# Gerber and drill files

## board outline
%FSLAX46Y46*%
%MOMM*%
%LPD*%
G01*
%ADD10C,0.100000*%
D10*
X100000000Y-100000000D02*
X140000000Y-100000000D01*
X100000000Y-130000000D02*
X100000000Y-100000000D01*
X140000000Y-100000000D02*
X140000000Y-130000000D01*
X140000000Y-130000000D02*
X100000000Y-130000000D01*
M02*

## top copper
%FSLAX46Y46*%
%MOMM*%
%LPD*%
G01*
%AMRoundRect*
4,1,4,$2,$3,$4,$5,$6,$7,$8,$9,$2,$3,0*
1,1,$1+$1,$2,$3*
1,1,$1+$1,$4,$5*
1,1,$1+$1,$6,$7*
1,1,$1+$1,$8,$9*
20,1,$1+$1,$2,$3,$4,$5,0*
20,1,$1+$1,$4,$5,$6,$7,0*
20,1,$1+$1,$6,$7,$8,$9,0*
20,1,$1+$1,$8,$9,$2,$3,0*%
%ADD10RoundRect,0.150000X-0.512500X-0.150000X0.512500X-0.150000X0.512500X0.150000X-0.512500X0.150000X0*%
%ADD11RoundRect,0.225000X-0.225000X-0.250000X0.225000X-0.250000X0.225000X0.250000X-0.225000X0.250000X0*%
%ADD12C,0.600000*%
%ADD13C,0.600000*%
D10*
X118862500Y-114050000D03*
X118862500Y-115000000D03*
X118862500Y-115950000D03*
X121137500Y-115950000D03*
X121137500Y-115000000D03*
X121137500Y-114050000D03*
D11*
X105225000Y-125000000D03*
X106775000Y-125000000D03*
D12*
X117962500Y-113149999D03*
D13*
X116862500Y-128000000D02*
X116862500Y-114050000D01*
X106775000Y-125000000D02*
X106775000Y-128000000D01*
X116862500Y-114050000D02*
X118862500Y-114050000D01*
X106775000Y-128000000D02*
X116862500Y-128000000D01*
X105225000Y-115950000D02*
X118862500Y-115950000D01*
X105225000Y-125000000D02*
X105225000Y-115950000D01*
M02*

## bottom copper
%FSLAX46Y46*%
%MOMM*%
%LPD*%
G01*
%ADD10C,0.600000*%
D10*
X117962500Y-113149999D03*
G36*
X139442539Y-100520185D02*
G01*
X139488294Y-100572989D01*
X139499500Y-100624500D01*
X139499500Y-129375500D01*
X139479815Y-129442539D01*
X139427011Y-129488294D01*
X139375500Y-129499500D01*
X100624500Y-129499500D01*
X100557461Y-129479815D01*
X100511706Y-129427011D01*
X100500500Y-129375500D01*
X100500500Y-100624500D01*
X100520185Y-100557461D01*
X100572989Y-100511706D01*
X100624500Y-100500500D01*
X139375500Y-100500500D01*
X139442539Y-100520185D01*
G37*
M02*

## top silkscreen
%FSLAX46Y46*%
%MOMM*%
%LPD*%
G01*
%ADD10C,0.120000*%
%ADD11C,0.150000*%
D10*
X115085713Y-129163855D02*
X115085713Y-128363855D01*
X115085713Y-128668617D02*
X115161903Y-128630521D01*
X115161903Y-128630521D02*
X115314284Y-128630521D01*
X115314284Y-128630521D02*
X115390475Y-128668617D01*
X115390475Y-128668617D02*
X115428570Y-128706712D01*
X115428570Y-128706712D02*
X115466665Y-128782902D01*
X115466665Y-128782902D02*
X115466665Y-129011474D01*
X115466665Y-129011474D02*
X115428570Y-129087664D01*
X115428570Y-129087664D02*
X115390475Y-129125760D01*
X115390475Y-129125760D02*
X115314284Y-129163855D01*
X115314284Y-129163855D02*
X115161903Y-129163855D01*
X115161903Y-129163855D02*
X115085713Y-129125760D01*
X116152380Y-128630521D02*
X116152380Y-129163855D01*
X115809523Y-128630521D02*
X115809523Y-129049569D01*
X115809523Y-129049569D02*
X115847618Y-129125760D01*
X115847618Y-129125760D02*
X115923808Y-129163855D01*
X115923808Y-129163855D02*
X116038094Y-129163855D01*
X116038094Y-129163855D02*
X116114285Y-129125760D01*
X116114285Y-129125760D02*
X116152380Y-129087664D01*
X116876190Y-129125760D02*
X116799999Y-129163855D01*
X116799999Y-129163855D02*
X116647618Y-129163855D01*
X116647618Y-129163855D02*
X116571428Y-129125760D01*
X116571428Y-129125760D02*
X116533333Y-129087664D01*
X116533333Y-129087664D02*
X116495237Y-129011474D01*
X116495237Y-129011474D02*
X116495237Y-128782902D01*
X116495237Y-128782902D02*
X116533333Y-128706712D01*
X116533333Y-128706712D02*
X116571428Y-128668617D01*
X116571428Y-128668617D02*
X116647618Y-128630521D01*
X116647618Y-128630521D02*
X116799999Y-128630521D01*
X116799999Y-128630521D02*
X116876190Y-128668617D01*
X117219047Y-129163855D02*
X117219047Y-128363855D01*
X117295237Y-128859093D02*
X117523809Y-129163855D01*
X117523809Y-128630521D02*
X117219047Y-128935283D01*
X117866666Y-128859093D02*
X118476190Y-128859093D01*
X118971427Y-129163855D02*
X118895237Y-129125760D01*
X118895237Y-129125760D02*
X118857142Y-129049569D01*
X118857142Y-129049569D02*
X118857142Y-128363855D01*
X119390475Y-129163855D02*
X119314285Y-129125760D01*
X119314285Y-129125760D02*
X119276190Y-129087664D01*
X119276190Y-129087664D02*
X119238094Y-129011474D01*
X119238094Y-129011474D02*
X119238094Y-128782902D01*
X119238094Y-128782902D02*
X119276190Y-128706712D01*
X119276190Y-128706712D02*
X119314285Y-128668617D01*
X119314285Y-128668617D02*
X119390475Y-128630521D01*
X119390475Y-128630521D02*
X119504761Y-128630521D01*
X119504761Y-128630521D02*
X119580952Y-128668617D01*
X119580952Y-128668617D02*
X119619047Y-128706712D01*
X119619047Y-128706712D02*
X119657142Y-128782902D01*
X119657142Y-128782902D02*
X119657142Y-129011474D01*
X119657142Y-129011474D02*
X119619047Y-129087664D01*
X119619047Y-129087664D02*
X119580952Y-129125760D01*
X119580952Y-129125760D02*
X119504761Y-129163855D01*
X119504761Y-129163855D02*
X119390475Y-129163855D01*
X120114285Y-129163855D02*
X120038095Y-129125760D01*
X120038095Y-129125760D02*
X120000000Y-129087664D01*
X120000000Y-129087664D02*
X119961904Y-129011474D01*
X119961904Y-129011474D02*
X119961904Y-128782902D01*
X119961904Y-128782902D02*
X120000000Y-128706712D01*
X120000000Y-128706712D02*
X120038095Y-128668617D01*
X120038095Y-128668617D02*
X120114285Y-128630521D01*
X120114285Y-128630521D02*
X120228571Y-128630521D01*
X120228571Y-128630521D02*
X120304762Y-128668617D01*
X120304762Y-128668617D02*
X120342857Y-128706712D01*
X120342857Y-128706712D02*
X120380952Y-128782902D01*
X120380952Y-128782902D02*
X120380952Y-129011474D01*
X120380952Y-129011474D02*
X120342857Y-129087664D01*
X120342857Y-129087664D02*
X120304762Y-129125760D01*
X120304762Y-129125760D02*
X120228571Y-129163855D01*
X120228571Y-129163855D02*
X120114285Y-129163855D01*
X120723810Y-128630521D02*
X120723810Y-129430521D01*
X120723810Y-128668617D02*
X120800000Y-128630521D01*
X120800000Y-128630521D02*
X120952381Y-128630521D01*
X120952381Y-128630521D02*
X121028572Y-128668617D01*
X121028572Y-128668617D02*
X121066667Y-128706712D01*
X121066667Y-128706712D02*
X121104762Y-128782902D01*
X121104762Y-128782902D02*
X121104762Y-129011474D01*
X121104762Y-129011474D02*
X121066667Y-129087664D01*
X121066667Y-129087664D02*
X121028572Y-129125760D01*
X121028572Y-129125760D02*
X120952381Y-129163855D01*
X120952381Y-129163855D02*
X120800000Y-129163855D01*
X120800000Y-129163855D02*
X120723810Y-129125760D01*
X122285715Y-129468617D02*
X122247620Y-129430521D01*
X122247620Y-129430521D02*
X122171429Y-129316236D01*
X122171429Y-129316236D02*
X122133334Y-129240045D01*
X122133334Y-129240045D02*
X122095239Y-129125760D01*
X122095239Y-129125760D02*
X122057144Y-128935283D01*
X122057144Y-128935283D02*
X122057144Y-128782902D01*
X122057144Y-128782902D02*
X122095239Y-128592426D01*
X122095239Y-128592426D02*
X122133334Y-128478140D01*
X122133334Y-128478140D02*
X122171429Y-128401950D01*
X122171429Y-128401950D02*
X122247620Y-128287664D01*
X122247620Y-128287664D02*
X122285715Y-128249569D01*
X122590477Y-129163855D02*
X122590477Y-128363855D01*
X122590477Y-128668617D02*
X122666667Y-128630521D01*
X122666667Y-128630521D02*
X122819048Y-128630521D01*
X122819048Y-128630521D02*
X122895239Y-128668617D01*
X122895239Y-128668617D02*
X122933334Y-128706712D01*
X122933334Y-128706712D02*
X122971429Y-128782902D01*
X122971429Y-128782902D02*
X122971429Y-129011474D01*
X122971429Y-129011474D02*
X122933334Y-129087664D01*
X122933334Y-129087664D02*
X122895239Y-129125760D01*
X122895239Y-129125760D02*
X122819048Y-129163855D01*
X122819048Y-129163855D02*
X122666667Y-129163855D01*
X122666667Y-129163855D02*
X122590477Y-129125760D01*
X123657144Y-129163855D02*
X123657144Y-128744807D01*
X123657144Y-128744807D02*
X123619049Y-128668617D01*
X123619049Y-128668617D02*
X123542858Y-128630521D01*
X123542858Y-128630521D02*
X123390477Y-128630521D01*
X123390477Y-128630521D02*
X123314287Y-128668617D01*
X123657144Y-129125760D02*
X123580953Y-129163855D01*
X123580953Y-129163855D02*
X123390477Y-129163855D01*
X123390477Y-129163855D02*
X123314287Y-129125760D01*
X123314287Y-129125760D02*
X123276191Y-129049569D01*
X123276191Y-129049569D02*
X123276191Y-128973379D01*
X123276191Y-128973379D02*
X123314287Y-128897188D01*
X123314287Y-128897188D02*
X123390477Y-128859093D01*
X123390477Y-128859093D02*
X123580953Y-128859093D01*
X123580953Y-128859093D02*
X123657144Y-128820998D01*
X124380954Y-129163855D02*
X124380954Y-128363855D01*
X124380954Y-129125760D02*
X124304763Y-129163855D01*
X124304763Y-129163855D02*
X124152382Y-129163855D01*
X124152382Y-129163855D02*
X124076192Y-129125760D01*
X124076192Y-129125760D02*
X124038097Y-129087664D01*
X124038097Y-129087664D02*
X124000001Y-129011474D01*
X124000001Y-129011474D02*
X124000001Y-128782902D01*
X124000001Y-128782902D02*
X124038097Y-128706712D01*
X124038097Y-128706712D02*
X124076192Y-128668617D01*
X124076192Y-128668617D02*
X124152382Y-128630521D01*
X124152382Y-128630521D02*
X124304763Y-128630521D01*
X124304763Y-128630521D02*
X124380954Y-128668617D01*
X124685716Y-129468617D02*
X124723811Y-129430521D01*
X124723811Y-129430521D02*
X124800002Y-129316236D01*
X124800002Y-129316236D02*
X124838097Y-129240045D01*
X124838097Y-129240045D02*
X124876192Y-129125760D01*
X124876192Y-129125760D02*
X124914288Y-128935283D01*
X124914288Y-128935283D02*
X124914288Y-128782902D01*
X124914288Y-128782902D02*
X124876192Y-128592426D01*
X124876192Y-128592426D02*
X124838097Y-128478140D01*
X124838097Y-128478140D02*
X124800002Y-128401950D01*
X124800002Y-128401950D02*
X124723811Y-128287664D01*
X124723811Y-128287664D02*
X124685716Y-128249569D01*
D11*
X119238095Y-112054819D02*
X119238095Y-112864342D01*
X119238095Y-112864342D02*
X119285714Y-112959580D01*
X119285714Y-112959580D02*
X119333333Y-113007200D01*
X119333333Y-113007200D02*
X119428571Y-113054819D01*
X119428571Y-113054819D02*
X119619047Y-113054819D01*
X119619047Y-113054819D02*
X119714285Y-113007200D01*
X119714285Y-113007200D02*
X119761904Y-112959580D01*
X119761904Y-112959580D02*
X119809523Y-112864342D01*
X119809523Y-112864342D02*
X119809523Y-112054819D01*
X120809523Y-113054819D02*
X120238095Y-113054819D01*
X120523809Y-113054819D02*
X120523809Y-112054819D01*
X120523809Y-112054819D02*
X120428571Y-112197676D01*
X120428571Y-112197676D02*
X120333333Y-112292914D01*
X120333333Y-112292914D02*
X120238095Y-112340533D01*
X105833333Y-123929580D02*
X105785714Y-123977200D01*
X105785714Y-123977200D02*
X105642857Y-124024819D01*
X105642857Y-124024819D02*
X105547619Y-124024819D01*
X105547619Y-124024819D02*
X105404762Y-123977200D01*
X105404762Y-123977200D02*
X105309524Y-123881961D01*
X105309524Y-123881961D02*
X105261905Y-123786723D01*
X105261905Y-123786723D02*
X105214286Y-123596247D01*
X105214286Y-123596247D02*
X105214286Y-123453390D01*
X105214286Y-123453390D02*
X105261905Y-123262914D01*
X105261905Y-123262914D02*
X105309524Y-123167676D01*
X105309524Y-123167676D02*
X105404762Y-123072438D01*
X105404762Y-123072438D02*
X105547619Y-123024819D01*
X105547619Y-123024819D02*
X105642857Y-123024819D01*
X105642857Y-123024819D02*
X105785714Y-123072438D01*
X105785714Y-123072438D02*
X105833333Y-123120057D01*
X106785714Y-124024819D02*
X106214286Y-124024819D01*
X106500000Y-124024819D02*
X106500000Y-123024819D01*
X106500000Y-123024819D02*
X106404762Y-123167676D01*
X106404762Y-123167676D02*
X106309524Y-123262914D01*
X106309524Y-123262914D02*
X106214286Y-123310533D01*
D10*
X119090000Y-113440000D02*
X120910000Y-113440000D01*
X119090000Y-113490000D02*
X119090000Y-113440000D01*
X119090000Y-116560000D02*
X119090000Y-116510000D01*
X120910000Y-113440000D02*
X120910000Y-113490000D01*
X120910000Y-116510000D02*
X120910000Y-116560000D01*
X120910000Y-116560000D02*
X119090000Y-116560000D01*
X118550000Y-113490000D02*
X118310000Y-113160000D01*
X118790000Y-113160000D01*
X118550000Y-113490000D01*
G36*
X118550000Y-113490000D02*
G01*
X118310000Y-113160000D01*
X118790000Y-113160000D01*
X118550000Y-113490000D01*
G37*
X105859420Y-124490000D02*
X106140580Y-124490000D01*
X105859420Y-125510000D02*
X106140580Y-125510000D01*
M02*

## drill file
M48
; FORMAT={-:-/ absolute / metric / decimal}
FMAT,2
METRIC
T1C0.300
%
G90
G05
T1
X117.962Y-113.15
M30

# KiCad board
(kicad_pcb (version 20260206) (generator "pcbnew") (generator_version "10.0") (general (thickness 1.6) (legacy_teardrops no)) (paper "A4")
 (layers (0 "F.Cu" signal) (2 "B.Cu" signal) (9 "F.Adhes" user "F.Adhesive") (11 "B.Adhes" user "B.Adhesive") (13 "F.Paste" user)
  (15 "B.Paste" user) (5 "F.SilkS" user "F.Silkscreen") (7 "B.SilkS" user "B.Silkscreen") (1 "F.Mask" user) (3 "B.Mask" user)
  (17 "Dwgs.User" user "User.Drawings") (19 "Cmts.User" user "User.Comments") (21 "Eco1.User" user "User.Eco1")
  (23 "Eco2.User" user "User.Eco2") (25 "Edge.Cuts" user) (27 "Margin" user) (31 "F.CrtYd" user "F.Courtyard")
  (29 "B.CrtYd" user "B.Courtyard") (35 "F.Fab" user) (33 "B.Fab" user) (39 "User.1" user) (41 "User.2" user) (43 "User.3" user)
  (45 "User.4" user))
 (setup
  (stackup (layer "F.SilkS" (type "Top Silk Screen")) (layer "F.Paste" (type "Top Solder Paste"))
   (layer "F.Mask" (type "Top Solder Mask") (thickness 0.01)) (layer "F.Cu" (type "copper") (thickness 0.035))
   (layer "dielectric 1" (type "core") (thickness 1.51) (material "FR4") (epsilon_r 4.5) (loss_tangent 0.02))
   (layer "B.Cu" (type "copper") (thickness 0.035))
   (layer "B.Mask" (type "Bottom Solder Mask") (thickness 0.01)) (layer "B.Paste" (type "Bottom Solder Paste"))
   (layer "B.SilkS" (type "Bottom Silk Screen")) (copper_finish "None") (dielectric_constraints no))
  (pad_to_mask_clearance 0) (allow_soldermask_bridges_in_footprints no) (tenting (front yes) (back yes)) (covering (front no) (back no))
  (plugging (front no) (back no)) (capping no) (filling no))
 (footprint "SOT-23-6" (layer "F.Cu") (at 120 115)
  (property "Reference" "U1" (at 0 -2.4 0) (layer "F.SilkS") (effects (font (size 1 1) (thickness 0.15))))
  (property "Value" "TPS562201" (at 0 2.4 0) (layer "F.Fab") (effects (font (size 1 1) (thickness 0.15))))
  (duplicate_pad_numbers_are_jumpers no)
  (fp_line (start -0.91 -1.56) (end 0.91 -1.56) (stroke (width 0.12) (type solid)) (layer "F.SilkS"))
  (fp_line (start -0.91 -1.51) (end -0.91 -1.56) (stroke (width 0.12) (type solid)) (layer "F.SilkS"))
  (fp_line (start -0.91 1.56) (end -0.91 1.51) (stroke (width 0.12) (type solid)) (layer "F.SilkS"))
  (fp_line (start 0.91 -1.56) (end 0.91 -1.51) (stroke (width 0.12) (type solid)) (layer "F.SilkS"))
  (fp_line (start 0.91 1.51) (end 0.91 1.56) (stroke (width 0.12) (type solid)) (layer "F.SilkS"))
  (fp_line (start 0.91 1.56) (end -0.91 1.56) (stroke (width 0.12) (type solid)) (layer "F.SilkS"))
  (fp_poly (pts (xy -1.45 -1.51) (xy -1.69 -1.84) (xy -1.21 -1.84)) (stroke (width 0.12) (type solid)) (fill yes) (layer "F.SilkS"))
  (pad "1" smd roundrect (at -1.1375 -0.95) (size 1.325 0.6) (layers "F.Cu" "F.Mask" "F.Paste") (roundrect_rratio 0.25) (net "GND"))
  (pad "2" smd roundrect (at -1.1375 0) (size 1.325 0.6) (layers "F.Cu" "F.Mask" "F.Paste") (roundrect_rratio 0.25) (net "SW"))
  (pad "3" smd roundrect (at -1.1375 0.95) (size 1.325 0.6) (layers "F.Cu" "F.Mask" "F.Paste") (roundrect_rratio 0.25) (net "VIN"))
  (pad "4" smd roundrect (at 1.1375 0.95) (size 1.325 0.6) (layers "F.Cu" "F.Mask" "F.Paste") (roundrect_rratio 0.25) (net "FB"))
  (pad "5" smd roundrect (at 1.1375 0) (size 1.325 0.6) (layers "F.Cu" "F.Mask" "F.Paste") (roundrect_rratio 0.25) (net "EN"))
  (pad "6" smd roundrect (at 1.1375 -0.95) (size 1.325 0.6) (layers "F.Cu" "F.Mask" "F.Paste") (roundrect_rratio 0.25) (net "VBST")))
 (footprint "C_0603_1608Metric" (layer "F.Cu") (at 106 125)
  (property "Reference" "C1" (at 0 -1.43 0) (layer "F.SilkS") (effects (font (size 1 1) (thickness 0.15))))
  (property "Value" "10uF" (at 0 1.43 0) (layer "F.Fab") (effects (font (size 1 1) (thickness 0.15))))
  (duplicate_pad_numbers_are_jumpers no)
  (fp_line (start -0.14058 -0.51) (end 0.14058 -0.51) (stroke (width 0.12) (type solid)) (layer "F.SilkS"))
  (fp_line (start -0.14058 0.51) (end 0.14058 0.51) (stroke (width 0.12) (type solid)) (layer "F.SilkS"))
  (pad "1" smd roundrect (at -0.775 0) (size 0.9 0.95) (layers "F.Cu" "F.Mask" "F.Paste") (roundrect_rratio 0.25) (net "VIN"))
  (pad "2" smd roundrect (at 0.775 0) (size 0.9 0.95) (layers "F.Cu" "F.Mask" "F.Paste") (roundrect_rratio 0.25) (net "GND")))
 (gr_line (start 100 100) (end 140 100) (stroke (width 0.1) (type default)) (layer "Edge.Cuts"))
 (gr_line (start 100 130) (end 100 100) (stroke (width 0.1) (type default)) (layer "Edge.Cuts"))
 (gr_line (start 140 100) (end 140 130) (stroke (width 0.1) (type default)) (layer "Edge.Cuts"))
 (gr_line (start 140 130) (end 100 130) (stroke (width 0.1) (type default)) (layer "Edge.Cuts"))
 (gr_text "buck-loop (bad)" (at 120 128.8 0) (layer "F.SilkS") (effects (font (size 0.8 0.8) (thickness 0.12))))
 (segment (start 116.8625 128) (end 116.8625 114.05) (width 0.6) (layer "F.Cu") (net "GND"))
 (segment (start 106.775 125) (end 106.775 128) (width 0.6) (layer "F.Cu") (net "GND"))
 (segment (start 116.8625 114.05) (end 118.8625 114.05) (width 0.6) (layer "F.Cu") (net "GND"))
 (segment (start 106.775 128) (end 116.8625 128) (width 0.6) (layer "F.Cu") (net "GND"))
 (via (at 117.9625 113.149999) (size 0.6) (drill 0.3) (layers "F.Cu" "B.Cu") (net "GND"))
 (segment (start 105.225 115.95) (end 118.8625 115.95) (width 0.6) (layer "F.Cu") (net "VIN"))
 (segment (start 105.225 125) (end 105.225 115.95) (width 0.6) (layer "F.Cu") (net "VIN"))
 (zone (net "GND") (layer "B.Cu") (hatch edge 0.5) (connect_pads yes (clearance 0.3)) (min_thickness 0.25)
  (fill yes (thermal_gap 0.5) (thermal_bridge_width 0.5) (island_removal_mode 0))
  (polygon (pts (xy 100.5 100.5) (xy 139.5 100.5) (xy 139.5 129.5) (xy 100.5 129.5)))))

